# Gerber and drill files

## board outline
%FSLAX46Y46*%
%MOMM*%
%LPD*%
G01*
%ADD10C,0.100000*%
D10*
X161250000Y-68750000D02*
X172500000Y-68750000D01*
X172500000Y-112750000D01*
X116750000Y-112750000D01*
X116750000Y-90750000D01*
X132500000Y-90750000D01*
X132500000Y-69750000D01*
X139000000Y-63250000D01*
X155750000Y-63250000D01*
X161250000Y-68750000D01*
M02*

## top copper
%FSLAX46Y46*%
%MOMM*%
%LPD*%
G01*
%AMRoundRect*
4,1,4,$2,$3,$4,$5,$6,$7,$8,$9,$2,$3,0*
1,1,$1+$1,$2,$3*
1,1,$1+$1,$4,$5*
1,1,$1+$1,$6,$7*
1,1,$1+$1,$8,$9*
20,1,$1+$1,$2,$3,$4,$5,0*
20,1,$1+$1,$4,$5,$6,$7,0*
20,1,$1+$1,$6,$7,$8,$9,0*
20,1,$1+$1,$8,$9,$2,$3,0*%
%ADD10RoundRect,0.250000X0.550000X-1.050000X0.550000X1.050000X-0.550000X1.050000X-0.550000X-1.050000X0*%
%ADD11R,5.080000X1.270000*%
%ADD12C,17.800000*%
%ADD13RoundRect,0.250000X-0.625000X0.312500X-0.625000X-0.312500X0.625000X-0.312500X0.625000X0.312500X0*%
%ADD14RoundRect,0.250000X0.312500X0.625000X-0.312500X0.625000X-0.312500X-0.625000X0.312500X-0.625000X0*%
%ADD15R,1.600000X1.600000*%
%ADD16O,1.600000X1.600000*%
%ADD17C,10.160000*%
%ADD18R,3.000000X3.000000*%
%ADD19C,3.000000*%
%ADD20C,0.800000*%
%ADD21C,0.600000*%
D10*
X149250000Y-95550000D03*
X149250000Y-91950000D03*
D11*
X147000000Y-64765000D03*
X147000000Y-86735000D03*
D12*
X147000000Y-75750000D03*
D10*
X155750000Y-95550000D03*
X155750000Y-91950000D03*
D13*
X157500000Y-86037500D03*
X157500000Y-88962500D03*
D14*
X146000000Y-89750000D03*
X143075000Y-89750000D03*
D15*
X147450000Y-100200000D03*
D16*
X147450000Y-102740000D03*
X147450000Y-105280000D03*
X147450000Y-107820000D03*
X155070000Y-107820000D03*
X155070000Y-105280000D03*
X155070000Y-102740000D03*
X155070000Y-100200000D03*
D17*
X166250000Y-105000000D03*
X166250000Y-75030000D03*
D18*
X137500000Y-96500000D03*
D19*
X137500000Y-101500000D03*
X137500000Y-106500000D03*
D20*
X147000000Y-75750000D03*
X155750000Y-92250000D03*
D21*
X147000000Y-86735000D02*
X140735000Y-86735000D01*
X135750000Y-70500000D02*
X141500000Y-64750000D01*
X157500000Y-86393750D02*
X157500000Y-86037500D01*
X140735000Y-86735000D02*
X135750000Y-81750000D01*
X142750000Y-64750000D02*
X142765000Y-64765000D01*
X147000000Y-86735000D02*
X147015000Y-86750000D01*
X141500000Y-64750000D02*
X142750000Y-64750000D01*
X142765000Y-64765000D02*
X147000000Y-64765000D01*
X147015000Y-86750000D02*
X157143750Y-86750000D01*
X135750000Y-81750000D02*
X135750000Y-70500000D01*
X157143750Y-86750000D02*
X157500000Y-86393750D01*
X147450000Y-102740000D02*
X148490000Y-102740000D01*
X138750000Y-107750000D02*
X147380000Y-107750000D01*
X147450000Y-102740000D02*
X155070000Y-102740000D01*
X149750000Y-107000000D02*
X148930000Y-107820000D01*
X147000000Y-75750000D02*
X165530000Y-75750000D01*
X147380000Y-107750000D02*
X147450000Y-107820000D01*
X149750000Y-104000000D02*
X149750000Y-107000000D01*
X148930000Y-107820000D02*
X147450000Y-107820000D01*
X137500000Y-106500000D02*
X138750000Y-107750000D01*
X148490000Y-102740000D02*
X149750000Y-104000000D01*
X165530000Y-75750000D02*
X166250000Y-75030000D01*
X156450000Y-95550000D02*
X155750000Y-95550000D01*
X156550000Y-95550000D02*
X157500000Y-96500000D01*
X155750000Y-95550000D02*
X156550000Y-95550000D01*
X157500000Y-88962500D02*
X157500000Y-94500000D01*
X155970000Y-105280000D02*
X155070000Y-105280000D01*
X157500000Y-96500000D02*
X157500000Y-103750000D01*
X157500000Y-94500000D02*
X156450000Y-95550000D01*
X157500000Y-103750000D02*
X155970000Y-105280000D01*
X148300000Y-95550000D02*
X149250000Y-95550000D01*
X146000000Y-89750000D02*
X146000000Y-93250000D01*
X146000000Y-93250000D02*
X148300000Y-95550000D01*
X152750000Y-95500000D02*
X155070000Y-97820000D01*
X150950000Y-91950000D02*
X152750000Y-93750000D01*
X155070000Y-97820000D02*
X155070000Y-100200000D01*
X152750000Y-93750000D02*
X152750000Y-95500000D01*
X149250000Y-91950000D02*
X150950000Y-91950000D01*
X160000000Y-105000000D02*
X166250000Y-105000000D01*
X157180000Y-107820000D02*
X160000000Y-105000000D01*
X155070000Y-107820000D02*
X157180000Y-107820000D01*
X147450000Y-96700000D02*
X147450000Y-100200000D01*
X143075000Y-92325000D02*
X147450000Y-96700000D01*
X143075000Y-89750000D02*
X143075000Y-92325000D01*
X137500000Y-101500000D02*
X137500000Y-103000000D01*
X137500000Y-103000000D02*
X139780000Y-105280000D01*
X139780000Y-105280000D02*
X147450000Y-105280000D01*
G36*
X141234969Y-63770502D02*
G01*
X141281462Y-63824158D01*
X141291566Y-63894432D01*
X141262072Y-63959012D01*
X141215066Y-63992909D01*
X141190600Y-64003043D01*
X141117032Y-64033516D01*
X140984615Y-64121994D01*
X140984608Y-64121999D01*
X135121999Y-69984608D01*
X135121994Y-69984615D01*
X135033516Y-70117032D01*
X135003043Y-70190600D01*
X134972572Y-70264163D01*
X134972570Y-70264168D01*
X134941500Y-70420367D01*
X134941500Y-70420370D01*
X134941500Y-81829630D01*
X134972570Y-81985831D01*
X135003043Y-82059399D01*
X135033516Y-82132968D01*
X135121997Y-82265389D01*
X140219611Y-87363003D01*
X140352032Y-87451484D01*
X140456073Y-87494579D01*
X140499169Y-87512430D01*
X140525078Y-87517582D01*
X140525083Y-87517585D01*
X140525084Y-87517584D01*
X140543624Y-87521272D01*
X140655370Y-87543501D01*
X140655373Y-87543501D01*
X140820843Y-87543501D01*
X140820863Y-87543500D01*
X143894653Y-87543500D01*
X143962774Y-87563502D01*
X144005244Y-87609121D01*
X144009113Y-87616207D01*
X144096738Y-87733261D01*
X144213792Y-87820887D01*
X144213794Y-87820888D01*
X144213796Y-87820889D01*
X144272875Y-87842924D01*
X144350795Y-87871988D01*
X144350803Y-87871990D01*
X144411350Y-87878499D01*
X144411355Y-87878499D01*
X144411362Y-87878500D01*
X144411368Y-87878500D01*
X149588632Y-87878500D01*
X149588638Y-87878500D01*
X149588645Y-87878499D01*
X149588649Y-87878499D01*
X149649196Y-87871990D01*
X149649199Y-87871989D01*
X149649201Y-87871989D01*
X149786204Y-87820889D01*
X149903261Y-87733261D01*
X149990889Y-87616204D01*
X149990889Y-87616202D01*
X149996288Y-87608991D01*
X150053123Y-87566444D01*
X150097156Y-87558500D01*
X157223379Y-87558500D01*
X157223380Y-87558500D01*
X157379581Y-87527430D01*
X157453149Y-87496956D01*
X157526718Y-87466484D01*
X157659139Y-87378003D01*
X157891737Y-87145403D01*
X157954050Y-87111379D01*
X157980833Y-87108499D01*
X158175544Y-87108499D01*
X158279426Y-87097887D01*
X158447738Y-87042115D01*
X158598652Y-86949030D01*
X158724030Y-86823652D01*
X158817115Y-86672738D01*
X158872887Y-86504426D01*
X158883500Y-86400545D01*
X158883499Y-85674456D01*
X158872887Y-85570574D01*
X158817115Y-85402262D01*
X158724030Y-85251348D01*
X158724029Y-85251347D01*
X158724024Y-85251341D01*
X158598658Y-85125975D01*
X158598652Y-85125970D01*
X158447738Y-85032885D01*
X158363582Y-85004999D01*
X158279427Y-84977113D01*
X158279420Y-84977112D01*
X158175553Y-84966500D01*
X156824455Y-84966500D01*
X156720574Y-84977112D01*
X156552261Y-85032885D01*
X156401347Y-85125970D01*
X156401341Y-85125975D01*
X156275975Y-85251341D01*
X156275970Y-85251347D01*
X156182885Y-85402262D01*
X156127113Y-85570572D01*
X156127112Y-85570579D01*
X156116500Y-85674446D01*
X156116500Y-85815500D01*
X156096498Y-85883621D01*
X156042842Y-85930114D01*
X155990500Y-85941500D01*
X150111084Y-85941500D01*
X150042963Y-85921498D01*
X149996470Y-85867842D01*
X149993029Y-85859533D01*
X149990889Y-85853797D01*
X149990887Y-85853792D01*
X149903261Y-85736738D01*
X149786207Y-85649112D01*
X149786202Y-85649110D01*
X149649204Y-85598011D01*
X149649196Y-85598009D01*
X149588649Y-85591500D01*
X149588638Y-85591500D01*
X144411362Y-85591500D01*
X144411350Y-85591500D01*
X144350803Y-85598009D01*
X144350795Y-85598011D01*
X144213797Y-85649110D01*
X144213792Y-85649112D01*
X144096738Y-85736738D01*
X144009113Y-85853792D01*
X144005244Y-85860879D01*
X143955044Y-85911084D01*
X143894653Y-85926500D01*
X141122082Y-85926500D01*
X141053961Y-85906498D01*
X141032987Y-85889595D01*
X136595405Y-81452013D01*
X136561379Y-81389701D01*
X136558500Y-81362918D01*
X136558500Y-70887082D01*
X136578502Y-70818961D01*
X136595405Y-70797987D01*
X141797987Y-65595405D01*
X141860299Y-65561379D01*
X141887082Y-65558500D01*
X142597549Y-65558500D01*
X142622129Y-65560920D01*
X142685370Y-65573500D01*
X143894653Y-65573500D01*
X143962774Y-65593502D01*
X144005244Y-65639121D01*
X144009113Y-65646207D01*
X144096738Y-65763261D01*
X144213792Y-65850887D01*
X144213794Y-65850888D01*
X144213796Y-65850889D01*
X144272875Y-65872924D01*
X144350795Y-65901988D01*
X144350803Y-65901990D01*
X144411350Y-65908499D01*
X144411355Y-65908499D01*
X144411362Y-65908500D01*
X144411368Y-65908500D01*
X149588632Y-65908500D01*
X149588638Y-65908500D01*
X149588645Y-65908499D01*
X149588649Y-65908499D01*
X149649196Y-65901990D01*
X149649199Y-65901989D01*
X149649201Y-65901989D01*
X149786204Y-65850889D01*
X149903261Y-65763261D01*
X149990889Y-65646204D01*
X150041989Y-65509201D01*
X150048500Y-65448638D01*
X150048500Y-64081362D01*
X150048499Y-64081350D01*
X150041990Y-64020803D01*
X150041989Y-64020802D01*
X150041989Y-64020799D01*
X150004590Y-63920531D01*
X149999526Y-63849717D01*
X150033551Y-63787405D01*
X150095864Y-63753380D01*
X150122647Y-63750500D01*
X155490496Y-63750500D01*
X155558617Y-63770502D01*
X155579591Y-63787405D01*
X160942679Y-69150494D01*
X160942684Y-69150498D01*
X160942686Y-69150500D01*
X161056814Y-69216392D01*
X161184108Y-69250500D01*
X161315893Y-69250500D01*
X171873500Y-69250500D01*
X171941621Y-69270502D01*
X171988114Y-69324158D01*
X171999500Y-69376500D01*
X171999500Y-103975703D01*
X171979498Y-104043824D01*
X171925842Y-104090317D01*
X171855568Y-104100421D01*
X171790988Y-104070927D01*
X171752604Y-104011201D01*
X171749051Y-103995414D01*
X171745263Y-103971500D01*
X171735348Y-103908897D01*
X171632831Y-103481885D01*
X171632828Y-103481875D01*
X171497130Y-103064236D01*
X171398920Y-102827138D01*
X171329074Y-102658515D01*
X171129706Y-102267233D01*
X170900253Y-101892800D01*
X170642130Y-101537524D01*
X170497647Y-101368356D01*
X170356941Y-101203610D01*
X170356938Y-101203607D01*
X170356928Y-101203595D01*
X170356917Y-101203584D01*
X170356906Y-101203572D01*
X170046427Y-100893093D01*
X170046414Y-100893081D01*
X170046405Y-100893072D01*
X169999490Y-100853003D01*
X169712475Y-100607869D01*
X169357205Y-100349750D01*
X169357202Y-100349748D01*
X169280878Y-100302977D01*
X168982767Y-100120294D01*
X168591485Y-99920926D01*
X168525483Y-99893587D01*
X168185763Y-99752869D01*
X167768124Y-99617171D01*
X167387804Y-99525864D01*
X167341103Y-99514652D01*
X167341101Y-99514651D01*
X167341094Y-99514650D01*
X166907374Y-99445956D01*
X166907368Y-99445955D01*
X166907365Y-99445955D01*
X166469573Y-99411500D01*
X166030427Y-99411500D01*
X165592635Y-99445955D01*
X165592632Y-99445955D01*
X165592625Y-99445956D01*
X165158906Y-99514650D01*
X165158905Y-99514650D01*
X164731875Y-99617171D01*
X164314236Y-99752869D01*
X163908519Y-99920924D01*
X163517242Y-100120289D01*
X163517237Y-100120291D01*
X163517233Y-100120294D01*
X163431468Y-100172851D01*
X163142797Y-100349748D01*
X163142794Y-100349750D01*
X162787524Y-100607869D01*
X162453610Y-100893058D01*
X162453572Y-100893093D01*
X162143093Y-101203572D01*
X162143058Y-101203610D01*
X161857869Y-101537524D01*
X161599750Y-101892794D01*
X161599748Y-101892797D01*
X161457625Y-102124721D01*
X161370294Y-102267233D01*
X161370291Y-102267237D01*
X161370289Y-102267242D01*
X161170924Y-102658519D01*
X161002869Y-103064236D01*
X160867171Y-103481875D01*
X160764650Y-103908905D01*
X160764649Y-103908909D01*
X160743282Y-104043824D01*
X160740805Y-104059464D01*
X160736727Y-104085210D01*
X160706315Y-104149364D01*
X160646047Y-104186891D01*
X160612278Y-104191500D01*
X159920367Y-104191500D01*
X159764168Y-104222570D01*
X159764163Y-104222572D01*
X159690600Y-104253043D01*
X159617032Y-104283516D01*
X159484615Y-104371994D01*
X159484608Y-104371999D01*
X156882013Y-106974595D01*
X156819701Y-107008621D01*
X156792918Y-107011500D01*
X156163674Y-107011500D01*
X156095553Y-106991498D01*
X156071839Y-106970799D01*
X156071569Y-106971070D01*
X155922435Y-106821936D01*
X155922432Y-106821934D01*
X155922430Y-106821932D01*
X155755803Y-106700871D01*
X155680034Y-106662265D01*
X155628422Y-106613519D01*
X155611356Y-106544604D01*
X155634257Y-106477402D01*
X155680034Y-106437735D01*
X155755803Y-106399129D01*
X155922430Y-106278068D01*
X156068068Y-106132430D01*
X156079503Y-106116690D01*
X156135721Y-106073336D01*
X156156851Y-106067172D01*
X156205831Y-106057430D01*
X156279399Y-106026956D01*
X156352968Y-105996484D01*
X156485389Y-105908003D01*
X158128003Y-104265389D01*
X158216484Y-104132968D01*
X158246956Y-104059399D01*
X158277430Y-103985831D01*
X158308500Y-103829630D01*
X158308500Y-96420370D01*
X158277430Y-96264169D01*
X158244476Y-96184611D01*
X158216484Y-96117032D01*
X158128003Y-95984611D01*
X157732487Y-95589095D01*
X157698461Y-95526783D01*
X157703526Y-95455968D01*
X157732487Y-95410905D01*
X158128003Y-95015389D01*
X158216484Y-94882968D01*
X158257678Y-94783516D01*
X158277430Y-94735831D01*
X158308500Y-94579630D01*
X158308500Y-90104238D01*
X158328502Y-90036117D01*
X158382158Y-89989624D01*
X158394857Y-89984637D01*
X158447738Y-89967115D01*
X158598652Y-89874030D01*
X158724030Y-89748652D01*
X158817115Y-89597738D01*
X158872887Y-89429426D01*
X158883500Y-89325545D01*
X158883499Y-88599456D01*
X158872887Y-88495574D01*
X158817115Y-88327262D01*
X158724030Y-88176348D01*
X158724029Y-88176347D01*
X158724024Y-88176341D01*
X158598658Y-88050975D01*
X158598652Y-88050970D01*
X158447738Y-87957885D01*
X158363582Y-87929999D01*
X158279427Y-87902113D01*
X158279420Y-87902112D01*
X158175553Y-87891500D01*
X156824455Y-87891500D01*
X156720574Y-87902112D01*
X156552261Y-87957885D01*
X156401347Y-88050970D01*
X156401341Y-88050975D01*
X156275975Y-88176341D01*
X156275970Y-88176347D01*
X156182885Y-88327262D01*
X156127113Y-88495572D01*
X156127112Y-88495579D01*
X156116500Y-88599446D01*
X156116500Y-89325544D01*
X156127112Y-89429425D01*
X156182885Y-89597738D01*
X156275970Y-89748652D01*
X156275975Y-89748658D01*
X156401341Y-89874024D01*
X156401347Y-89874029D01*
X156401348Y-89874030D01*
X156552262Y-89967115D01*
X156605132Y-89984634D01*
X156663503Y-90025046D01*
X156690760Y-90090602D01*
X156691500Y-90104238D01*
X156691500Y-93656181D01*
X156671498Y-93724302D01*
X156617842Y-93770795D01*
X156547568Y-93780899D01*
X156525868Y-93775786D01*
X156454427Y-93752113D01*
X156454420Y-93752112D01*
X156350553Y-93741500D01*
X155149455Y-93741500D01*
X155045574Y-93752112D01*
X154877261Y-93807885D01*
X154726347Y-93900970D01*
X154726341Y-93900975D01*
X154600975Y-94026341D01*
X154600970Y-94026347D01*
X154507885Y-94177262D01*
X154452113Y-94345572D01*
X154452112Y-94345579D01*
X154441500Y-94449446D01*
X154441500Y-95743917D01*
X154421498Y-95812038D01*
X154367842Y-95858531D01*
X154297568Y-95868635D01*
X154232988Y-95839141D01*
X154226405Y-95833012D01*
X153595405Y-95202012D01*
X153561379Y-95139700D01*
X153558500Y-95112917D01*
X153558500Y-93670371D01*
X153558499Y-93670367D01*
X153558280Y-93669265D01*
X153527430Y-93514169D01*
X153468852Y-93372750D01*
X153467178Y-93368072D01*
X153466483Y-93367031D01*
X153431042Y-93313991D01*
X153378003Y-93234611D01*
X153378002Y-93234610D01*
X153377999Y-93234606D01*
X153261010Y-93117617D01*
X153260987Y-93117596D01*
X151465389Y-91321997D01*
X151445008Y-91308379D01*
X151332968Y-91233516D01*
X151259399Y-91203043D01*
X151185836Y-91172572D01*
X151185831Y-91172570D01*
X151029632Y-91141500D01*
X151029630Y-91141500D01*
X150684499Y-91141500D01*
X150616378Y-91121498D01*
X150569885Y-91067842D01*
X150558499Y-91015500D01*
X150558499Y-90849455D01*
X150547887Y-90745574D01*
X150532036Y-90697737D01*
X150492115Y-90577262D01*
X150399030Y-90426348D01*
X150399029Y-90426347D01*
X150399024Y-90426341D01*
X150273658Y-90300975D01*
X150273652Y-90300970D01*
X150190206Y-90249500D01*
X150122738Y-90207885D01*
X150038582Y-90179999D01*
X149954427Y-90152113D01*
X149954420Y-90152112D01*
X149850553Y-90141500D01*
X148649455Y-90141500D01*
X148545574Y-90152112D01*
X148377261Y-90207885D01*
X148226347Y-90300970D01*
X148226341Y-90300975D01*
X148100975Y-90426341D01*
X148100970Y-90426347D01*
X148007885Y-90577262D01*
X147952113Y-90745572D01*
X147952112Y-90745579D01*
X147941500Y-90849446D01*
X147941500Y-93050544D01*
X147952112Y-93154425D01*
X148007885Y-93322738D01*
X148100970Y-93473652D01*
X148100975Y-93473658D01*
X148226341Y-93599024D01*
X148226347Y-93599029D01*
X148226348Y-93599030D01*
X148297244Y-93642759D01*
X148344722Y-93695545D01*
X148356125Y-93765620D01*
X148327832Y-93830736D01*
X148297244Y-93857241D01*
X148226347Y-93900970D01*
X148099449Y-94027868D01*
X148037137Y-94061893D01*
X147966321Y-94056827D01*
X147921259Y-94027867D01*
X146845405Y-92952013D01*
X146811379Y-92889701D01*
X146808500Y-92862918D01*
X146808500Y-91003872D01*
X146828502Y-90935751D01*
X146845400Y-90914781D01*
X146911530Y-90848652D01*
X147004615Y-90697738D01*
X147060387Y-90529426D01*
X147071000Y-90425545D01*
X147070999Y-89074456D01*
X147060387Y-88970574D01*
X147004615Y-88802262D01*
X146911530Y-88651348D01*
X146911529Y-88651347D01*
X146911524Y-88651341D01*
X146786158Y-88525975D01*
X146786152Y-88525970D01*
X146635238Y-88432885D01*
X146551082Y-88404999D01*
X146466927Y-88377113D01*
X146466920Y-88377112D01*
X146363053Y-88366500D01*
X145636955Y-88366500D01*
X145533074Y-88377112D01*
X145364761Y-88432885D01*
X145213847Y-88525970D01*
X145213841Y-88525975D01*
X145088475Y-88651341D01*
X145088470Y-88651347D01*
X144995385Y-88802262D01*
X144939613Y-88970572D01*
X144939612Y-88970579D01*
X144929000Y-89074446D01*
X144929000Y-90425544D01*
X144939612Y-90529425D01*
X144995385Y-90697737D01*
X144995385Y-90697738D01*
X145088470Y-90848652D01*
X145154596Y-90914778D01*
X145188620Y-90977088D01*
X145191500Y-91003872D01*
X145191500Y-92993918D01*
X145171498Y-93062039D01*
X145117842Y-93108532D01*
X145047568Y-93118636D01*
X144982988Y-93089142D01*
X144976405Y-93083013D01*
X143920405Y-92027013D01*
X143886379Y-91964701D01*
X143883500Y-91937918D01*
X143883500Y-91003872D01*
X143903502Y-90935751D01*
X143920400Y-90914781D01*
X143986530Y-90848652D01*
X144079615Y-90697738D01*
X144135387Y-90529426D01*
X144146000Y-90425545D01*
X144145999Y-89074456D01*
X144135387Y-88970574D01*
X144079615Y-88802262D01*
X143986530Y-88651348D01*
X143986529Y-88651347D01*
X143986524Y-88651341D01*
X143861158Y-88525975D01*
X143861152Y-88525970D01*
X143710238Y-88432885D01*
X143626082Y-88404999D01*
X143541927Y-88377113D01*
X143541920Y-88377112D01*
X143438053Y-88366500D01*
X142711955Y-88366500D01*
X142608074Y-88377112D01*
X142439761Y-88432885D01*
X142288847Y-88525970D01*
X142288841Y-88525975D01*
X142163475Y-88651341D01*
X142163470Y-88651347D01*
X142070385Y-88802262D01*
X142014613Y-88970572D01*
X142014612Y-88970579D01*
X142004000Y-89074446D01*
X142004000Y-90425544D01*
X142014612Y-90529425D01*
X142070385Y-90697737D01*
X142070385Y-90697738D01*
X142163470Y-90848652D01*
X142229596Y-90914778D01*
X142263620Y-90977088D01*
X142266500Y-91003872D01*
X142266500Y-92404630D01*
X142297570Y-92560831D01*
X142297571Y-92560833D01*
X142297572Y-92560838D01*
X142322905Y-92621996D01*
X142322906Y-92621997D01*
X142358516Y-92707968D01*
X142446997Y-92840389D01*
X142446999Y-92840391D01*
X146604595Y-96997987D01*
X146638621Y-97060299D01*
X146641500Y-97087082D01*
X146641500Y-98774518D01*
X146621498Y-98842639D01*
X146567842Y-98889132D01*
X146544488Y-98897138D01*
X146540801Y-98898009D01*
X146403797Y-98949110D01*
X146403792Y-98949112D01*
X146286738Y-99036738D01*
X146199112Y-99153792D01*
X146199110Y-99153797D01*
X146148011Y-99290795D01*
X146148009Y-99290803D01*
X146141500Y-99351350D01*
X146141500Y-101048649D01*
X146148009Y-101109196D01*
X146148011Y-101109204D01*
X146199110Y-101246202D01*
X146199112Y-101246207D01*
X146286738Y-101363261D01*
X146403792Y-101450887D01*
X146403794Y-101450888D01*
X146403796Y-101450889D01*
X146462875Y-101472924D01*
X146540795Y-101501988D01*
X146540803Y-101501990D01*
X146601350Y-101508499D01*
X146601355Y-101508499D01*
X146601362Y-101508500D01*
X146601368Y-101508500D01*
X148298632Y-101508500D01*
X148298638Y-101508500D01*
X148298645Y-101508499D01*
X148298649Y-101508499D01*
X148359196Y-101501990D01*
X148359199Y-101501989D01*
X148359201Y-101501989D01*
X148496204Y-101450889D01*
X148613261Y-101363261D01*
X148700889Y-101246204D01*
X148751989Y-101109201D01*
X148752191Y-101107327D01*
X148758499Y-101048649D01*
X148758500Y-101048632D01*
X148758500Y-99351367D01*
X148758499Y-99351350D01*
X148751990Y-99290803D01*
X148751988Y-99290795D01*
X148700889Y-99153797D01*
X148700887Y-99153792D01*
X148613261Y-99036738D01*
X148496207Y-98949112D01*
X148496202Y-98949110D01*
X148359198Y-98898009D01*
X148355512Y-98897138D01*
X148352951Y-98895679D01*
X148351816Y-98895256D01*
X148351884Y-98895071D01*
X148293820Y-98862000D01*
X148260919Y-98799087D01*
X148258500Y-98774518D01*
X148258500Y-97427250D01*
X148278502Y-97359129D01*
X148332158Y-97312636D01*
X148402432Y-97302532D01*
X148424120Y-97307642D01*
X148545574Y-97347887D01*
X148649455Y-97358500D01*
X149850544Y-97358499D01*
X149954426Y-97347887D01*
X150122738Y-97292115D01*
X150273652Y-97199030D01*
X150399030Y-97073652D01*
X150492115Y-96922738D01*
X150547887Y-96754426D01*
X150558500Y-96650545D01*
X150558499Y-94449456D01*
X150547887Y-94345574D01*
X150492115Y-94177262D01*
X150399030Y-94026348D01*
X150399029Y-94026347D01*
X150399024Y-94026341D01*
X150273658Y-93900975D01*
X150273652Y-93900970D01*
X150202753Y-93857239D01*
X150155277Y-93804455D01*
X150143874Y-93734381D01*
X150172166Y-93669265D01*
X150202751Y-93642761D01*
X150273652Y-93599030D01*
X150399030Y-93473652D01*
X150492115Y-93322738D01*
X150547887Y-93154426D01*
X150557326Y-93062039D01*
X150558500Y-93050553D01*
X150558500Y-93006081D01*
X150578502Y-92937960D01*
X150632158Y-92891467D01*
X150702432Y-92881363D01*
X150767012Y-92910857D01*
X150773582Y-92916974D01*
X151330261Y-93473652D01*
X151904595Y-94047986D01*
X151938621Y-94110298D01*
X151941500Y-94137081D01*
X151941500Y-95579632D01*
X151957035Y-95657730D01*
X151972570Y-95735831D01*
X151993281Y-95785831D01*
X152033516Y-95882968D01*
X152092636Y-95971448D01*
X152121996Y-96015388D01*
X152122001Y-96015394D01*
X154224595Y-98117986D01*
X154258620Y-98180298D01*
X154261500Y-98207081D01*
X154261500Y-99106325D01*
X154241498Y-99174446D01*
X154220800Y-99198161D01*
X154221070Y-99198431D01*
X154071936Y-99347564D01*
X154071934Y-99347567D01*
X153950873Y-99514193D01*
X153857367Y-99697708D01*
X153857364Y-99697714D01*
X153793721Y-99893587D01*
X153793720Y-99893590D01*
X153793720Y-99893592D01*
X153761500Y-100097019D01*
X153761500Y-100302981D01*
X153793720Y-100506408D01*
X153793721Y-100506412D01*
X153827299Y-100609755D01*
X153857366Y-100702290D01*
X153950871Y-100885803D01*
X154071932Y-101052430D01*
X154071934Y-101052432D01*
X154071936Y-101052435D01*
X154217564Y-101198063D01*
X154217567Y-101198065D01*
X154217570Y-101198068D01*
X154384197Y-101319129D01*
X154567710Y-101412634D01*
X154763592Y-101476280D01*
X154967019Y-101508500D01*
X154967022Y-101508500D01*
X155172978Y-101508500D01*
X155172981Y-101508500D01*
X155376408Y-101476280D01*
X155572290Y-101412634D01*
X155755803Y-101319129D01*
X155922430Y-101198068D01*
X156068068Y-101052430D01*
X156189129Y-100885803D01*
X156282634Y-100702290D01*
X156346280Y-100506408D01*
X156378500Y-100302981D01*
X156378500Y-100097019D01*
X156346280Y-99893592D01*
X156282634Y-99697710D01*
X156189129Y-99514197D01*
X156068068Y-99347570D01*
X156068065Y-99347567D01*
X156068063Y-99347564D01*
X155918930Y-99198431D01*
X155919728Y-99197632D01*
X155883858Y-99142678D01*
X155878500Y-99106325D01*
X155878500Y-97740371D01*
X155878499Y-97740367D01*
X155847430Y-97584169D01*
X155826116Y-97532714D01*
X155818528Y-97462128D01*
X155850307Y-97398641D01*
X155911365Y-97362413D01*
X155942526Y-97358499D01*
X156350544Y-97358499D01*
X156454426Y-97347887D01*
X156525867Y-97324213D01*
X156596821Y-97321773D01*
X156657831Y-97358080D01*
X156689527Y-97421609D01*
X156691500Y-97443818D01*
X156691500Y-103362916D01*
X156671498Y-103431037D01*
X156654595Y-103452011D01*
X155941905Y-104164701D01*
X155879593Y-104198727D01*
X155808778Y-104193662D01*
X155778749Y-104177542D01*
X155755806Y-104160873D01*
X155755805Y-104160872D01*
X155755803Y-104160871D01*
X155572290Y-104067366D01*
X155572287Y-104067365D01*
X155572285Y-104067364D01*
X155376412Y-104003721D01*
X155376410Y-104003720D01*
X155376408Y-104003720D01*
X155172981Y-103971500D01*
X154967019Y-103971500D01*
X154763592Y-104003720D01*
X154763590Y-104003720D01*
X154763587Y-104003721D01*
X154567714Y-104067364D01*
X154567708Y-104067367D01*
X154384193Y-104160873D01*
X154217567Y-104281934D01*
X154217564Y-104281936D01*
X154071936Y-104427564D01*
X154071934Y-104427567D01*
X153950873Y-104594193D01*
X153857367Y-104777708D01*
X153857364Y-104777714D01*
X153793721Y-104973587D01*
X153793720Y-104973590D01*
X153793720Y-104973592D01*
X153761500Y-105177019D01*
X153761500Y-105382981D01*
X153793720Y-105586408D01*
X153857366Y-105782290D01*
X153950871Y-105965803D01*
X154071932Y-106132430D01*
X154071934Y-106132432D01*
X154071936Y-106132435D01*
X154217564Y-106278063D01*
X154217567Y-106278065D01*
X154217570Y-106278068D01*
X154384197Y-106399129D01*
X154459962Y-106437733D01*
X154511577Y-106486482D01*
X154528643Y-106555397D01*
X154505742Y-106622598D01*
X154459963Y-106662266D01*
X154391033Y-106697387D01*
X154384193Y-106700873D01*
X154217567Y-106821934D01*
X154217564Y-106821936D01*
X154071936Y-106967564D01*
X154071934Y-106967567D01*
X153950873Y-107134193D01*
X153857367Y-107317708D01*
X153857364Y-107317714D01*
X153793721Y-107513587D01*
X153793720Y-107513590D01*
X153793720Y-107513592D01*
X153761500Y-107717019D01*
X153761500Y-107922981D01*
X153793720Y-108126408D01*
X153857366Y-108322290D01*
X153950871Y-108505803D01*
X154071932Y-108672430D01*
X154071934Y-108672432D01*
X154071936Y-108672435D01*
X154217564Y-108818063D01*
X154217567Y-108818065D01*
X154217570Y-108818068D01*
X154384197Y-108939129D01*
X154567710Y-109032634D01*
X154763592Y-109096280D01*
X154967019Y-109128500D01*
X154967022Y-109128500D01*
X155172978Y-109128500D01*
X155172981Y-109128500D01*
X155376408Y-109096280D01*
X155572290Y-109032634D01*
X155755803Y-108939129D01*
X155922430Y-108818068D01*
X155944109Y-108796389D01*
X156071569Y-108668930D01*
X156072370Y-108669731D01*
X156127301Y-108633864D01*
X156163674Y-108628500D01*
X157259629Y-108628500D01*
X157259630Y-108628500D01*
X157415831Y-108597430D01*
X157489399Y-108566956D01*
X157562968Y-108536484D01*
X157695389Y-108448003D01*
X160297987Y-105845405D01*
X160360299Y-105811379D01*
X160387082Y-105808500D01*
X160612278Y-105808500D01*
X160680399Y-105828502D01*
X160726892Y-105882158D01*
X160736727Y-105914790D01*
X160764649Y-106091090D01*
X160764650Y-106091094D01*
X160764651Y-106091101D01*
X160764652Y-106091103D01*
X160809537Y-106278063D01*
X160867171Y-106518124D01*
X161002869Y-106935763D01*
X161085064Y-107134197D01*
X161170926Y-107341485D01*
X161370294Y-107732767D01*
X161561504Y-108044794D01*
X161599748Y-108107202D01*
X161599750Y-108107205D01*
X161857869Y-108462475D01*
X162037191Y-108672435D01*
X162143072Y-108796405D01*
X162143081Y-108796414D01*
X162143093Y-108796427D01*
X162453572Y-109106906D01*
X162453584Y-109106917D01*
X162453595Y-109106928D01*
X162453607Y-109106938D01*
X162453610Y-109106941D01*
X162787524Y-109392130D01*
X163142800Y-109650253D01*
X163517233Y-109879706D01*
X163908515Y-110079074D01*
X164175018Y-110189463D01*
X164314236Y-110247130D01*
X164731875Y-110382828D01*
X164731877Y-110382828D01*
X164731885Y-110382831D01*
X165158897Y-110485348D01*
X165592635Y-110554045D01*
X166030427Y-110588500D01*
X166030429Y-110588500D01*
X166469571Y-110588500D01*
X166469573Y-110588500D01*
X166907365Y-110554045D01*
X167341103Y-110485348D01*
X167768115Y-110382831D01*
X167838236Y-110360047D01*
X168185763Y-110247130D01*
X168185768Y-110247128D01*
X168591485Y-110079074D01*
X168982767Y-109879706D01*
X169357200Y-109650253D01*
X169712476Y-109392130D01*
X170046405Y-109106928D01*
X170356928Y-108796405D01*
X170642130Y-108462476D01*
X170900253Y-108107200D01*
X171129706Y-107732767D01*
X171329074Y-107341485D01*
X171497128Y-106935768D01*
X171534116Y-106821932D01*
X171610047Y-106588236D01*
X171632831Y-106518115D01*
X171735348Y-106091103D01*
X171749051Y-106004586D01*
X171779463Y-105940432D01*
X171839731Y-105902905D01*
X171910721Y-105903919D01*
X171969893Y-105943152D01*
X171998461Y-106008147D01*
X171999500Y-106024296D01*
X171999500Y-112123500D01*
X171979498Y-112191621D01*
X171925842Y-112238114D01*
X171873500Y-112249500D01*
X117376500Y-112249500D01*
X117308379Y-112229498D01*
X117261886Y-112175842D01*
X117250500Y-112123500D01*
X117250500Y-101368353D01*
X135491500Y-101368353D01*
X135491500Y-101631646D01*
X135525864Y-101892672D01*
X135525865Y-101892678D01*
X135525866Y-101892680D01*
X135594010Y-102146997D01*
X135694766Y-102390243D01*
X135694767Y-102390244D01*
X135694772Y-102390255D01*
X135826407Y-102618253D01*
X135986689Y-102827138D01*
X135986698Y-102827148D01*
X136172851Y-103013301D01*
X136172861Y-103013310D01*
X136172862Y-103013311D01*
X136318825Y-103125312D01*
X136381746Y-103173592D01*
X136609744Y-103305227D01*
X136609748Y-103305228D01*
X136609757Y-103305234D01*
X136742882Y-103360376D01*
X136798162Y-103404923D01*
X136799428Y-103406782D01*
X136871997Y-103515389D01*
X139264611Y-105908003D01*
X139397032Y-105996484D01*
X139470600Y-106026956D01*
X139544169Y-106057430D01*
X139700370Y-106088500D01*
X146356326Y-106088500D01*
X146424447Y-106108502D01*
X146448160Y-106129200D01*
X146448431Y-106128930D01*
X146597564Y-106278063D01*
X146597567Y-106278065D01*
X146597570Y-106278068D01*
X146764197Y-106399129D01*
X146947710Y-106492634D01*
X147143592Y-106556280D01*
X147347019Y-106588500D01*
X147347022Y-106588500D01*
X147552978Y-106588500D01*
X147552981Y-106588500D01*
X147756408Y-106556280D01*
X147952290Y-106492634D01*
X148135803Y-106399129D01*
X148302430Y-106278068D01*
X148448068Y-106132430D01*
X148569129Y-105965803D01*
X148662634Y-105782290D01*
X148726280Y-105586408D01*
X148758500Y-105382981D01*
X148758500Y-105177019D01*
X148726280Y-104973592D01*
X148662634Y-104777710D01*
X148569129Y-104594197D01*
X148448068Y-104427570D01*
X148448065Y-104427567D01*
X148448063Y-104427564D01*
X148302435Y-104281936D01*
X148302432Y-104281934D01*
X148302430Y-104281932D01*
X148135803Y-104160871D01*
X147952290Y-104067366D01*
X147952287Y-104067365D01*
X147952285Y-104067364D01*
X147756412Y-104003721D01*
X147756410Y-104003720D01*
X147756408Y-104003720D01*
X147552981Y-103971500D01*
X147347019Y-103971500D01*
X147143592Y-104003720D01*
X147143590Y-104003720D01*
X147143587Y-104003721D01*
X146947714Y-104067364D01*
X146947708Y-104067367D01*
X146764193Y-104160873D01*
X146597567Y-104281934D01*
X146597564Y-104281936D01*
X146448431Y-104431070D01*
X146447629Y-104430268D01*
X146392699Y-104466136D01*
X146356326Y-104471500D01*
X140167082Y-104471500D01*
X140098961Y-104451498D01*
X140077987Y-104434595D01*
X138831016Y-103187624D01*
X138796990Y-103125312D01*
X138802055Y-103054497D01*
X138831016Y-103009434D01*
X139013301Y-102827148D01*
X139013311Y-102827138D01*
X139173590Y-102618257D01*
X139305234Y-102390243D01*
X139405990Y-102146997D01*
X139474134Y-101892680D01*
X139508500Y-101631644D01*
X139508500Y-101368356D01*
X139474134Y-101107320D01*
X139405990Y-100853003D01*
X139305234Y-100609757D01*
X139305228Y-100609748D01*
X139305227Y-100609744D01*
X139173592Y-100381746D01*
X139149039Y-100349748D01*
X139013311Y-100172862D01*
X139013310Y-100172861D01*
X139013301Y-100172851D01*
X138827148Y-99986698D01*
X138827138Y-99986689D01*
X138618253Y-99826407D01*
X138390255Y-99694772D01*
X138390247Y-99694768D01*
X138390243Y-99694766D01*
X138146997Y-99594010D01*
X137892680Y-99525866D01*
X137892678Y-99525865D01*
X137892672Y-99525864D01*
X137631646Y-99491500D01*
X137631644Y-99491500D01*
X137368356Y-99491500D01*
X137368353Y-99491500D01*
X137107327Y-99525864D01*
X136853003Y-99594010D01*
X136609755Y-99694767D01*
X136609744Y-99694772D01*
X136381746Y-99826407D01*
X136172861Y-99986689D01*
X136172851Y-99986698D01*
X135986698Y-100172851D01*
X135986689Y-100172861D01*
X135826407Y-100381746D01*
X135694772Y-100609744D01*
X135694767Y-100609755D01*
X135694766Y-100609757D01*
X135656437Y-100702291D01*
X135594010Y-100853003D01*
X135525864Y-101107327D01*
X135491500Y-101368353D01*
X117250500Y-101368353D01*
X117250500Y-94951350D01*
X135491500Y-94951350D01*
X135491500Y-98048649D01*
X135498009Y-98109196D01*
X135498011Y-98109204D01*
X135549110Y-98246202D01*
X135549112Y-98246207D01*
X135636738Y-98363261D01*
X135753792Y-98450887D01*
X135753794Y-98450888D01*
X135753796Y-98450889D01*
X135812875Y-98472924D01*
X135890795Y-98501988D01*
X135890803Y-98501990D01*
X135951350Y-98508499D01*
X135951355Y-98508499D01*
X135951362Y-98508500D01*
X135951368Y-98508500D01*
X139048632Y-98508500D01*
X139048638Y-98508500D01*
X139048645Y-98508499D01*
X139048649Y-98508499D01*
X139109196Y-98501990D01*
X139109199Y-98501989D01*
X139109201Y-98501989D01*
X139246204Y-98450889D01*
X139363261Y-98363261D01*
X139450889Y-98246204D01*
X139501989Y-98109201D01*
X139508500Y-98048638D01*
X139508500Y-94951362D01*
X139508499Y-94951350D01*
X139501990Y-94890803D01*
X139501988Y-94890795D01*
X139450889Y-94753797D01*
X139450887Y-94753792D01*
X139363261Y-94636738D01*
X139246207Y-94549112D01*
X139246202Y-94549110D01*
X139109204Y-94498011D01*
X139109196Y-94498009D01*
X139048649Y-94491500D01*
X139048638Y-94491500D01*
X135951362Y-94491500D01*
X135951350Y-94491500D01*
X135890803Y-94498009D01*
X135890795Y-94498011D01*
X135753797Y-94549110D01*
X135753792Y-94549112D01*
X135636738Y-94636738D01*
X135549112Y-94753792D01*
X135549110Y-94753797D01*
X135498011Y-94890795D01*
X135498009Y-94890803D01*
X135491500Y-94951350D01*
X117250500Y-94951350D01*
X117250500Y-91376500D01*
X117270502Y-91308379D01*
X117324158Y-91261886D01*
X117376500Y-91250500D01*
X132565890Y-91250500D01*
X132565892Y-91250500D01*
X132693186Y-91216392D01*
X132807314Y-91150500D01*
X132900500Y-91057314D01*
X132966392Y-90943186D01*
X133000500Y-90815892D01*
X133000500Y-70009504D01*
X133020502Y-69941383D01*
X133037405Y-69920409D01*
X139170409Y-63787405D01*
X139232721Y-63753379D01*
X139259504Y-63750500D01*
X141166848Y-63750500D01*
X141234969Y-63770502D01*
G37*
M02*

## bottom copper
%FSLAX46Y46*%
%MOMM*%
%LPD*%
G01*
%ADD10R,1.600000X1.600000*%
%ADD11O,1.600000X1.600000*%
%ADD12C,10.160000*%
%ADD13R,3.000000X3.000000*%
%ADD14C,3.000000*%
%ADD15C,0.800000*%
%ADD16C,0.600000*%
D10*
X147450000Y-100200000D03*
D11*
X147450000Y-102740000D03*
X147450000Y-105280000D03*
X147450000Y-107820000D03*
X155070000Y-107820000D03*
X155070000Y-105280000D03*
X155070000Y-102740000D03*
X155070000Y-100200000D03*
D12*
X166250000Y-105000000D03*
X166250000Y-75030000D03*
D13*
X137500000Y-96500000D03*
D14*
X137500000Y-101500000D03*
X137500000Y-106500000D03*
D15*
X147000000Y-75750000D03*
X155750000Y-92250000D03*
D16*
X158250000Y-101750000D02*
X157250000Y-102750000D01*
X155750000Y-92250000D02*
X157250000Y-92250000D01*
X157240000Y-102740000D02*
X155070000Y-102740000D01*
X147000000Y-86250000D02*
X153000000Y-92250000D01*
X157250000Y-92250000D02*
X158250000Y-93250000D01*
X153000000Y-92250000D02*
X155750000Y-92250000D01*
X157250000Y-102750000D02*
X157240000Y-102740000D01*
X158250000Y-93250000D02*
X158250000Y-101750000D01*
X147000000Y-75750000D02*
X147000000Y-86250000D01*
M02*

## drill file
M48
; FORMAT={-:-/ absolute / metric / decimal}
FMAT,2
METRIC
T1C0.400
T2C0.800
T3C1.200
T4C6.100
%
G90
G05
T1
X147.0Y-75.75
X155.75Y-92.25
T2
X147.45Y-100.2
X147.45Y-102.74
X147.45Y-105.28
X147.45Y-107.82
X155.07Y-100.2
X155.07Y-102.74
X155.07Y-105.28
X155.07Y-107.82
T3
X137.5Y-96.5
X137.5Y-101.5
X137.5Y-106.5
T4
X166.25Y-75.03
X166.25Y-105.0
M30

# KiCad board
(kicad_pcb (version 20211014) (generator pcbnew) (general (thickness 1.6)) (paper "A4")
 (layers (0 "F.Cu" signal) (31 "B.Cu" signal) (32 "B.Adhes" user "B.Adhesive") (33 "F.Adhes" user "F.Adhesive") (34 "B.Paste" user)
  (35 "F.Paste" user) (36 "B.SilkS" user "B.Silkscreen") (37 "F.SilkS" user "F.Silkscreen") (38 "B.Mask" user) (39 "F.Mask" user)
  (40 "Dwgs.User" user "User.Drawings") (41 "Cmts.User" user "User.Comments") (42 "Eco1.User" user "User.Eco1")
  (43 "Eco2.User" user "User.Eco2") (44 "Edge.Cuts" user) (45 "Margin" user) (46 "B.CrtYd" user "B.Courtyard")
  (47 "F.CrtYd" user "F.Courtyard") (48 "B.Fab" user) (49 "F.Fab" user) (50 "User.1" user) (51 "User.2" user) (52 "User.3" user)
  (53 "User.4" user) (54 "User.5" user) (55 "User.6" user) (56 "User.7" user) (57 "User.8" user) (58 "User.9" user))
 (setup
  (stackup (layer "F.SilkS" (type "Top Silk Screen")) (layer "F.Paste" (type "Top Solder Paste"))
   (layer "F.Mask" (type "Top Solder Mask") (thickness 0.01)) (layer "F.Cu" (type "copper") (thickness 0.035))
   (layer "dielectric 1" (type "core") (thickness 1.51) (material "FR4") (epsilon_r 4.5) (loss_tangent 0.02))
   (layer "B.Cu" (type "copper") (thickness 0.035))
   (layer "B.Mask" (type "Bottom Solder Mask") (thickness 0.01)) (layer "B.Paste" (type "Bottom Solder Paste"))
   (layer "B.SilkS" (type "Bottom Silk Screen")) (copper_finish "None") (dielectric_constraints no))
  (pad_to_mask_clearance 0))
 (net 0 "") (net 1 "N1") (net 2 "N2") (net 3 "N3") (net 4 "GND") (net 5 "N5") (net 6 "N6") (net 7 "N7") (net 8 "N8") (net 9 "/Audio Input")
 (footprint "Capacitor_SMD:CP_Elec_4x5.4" (layer "F.Cu") (at 149.25 93.75 90)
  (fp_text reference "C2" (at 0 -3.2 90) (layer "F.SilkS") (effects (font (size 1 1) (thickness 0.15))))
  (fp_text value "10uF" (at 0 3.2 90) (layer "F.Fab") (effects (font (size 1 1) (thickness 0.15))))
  (pad "1" smd roundrect (at -1.8 0 90) (size 2.6 1.6) (layers "F.Cu" "F.Paste" "F.Mask") (roundrect_rratio 0.15625) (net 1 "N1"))
  (pad "2" smd roundrect (at 1.8 0 90) (size 2.6 1.6) (layers "F.Cu" "F.Paste" "F.Mask") (roundrect_rratio 0.15625) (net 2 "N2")))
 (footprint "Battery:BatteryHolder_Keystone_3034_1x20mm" (layer "F.Cu") (at 147 75.75 90)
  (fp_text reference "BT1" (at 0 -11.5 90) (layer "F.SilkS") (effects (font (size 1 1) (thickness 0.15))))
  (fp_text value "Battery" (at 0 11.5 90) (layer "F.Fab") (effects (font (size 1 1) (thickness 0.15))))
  (pad "1" smd rect (at 10.985 0 90) (size 1.27 5.08) (layers "F.Cu" "F.Paste" "F.Mask") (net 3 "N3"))
  (pad "1" smd rect (at -10.985 0 90) (size 1.27 5.08) (layers "F.Cu" "F.Paste" "F.Mask") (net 3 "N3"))
  (pad "2" smd circle (at 0 0 90) (size 17.8 17.8) (layers "F.Cu" "F.Mask") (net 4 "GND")))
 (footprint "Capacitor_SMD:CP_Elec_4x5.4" (layer "F.Cu") (at 155.75 93.75 90)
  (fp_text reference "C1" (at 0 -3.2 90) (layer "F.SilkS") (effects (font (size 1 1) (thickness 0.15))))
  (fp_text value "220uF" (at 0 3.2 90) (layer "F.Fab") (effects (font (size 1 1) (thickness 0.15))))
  (pad "1" smd roundrect (at -1.8 0 90) (size 2.6 1.6) (layers "F.Cu" "F.Paste" "F.Mask") (roundrect_rratio 0.15625) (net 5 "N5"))
  (pad "2" smd roundrect (at 1.8 0 90) (size 2.6 1.6) (layers "F.Cu" "F.Paste" "F.Mask") (roundrect_rratio 0.15625) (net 4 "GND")))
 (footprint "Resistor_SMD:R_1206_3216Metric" (layer "F.Cu") (at 157.5 87.5 -90)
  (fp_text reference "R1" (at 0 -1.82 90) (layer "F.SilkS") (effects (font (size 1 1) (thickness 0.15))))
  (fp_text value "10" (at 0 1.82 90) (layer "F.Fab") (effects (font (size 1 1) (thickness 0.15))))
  (pad "1" smd roundrect (at -1.4625 0 270) (size 1.125 1.75) (layers "F.Cu" "F.Paste" "F.Mask") (roundrect_rratio 0.2222222222)
   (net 3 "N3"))
  (pad "2" smd roundrect (at 1.4625 0 270) (size 1.125 1.75) (layers "F.Cu" "F.Paste" "F.Mask") (roundrect_rratio 0.2222222222) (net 5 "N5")))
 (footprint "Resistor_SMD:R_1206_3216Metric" (layer "F.Cu") (at 144.5375 89.75 180)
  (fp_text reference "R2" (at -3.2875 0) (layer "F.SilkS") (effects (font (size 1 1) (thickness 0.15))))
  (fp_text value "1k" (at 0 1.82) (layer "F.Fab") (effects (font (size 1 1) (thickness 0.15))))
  (pad "1" smd roundrect (at -1.4625 0 180) (size 1.125 1.75) (layers "F.Cu" "F.Paste" "F.Mask") (roundrect_rratio 0.2222222222)
   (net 1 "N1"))
  (pad "2" smd roundrect (at 1.4625 0 180) (size 1.125 1.75) (layers "F.Cu" "F.Paste" "F.Mask") (roundrect_rratio 0.2222222222) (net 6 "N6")))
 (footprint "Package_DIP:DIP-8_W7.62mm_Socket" (layer "F.Cu") (at 147.45 100.2)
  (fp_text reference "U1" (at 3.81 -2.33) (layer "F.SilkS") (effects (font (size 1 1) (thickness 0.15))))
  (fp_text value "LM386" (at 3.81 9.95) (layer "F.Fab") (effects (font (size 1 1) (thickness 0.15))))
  (pad "1" thru_hole rect (at 0 0) (size 1.6 1.6) (drill 0.8) (layers *.Cu *.Mask) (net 6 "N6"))
  (pad "2" thru_hole oval (at 0 2.54) (size 1.6 1.6) (drill 0.8) (layers *.Cu *.Mask) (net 4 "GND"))
  (pad "3" thru_hole oval (at 0 5.08) (size 1.6 1.6) (drill 0.8) (layers *.Cu *.Mask) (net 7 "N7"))
  (pad "4" thru_hole oval (at 0 7.62) (size 1.6 1.6) (drill 0.8) (layers *.Cu *.Mask) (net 4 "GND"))
  (pad "5" thru_hole oval (at 7.62 7.62) (size 1.6 1.6) (drill 0.8) (layers *.Cu *.Mask) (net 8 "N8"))
  (pad "6" thru_hole oval (at 7.62 5.08) (size 1.6 1.6) (drill 0.8) (layers *.Cu *.Mask) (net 5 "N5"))
  (pad "7" thru_hole oval (at 7.62 2.54) (size 1.6 1.6) (drill 0.8) (layers *.Cu *.Mask) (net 4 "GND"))
  (pad "8" thru_hole oval (at 7.62 0) (size 1.6 1.6) (drill 0.8) (layers *.Cu *.Mask) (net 2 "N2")))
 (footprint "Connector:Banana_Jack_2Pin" (layer "F.Cu") (at 166.25 105 90)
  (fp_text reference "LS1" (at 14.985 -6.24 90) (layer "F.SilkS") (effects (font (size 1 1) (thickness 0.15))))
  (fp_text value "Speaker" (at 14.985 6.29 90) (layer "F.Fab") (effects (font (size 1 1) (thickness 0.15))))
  (pad "1" thru_hole circle (at 0 0 90) (size 10.16 10.16) (drill 6.1) (layers *.Cu *.Mask) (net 8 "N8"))
  (pad "2" thru_hole circle (at 29.97 0 90) (size 10.16 10.16) (drill 6.1) (layers *.Cu *.Mask) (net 4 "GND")))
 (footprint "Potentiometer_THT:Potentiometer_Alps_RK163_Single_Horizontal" (layer "F.Cu") (at 137.5 96.5)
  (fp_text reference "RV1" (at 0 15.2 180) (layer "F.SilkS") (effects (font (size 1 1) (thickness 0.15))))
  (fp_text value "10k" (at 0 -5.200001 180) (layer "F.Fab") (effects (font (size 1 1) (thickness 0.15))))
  (pad "1" thru_hole rect (at 0 0 180) (size 3 3) (drill 1.2) (layers *.Cu *.Mask) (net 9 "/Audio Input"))
  (pad "2" thru_hole circle (at 0 5 180) (size 3 3) (drill 1.2) (layers *.Cu *.Mask) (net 7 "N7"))
  (pad "3" thru_hole circle (at 0 10 180) (size 3 3) (drill 1.2) (layers *.Cu *.Mask) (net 4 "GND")))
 (gr_poly
  (pts (xy 161.25 68.75) (xy 172.5 68.75) (xy 172.5 112.75) (xy 116.75 112.75) (xy 116.75 90.75) (xy 132.5 90.75) (xy 132.5 69.75)
   (xy 139 63.25) (xy 155.75 63.25))
  (layer "Edge.Cuts") (width 0.1) (fill none))
 (segment (start 147 86.735) (end 140.735 86.735) (width 0.6) (layer "F.Cu") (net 3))
 (segment (start 135.75 70.5) (end 141.5 64.75) (width 0.6) (layer "F.Cu") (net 3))
 (segment (start 157.5 86.39375) (end 157.5 86.0375) (width 0.6) (layer "F.Cu") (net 3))
 (segment (start 140.735 86.735) (end 135.75 81.75) (width 0.6) (layer "F.Cu") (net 3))
 (segment (start 142.75 64.75) (end 142.765 64.765) (width 0.6) (layer "F.Cu") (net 3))
 (segment (start 147 86.735) (end 147.015 86.75) (width 0.6) (layer "F.Cu") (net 3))
 (segment (start 141.5 64.75) (end 142.75 64.75) (width 0.6) (layer "F.Cu") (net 3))
 (segment (start 142.765 64.765) (end 147 64.765) (width 0.6) (layer "F.Cu") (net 3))
 (segment (start 147.015 86.75) (end 157.14375 86.75) (width 0.6) (layer "F.Cu") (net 3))
 (segment (start 135.75 81.75) (end 135.75 70.5) (width 0.6) (layer "F.Cu") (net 3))
 (segment (start 157.14375 86.75) (end 157.5 86.39375) (width 0.6) (layer "F.Cu") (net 3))
 (segment (start 147.45 102.74) (end 148.49 102.74) (width 0.6) (layer "F.Cu") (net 4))
 (segment (start 138.75 107.75) (end 147.38 107.75) (width 0.6) (layer "F.Cu") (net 4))
 (segment (start 147.45 102.74) (end 155.07 102.74) (width 0.6) (layer "F.Cu") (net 4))
 (segment (start 149.75 107) (end 148.93 107.82) (width 0.6) (layer "F.Cu") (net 4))
 (segment (start 147 75.75) (end 165.53 75.75) (width 0.6) (layer "F.Cu") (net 4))
 (segment (start 147.38 107.75) (end 147.45 107.82) (width 0.6) (layer "F.Cu") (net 4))
 (segment (start 149.75 104) (end 149.75 107) (width 0.6) (layer "F.Cu") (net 4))
 (segment (start 148.93 107.82) (end 147.45 107.82) (width 0.6) (layer "F.Cu") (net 4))
 (segment (start 137.5 106.5) (end 138.75 107.75) (width 0.6) (layer "F.Cu") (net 4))
 (segment (start 148.49 102.74) (end 149.75 104) (width 0.6) (layer "F.Cu") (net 4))
 (segment (start 165.53 75.75) (end 166.25 75.03) (width 0.6) (layer "F.Cu") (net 4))
 (via (at 147 75.75) (size 0.8) (drill 0.4) (layers "F.Cu" "B.Cu") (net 4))
 (via (at 155.75 92.25) (size 0.8) (drill 0.4) (layers "F.Cu" "B.Cu") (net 4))
 (segment (start 158.25 101.75) (end 157.25 102.75) (width 0.6) (layer "B.Cu") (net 4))
 (segment (start 155.75 92.25) (end 157.25 92.25) (width 0.6) (layer "B.Cu") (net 4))
 (segment (start 157.24 102.74) (end 155.07 102.74) (width 0.6) (layer "B.Cu") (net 4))
 (segment (start 147 86.25) (end 153 92.25) (width 0.6) (layer "B.Cu") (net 4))
 (segment (start 157.25 92.25) (end 158.25 93.25) (width 0.6) (layer "B.Cu") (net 4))
 (segment (start 153 92.25) (end 155.75 92.25) (width 0.6) (layer "B.Cu") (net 4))
 (segment (start 157.25 102.75) (end 157.24 102.74) (width 0.6) (layer "B.Cu") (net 4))
 (segment (start 158.25 93.25) (end 158.25 101.75) (width 0.6) (layer "B.Cu") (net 4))
 (segment (start 147 75.75) (end 147 86.25) (width 0.6) (layer "B.Cu") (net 4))
 (segment (start 156.45 95.55) (end 155.75 95.55) (width 0.6) (layer "F.Cu") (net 5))
 (segment (start 156.55 95.55) (end 157.5 96.5) (width 0.6) (layer "F.Cu") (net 5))
 (segment (start 155.75 95.55) (end 156.55 95.55) (width 0.6) (layer "F.Cu") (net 5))
 (segment (start 157.5 88.9625) (end 157.5 94.5) (width 0.6) (layer "F.Cu") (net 5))
 (segment (start 155.97 105.28) (end 155.07 105.28) (width 0.6) (layer "F.Cu") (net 5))
 (segment (start 157.5 96.5) (end 157.5 103.75) (width 0.6) (layer "F.Cu") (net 5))
 (segment (start 157.5 94.5) (end 156.45 95.55) (width 0.6) (layer "F.Cu") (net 5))
 (segment (start 157.5 103.75) (end 155.97 105.28) (width 0.6) (layer "F.Cu") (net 5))
 (segment (start 148.3 95.55) (end 149.25 95.55) (width 0.6) (layer "F.Cu") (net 1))
 (segment (start 146 89.75) (end 146 93.25) (width 0.6) (layer "F.Cu") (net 1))
 (segment (start 146 93.25) (end 148.3 95.55) (width 0.6) (layer "F.Cu") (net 1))
 (segment (start 152.75 95.5) (end 155.07 97.82) (width 0.6) (layer "F.Cu") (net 2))
 (segment (start 150.95 91.95) (end 152.75 93.75) (width 0.6) (layer "F.Cu") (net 2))
 (segment (start 155.07 97.82) (end 155.07 100.2) (width 0.6) (layer "F.Cu") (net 2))
 (segment (start 152.75 93.75) (end 152.75 95.5) (width 0.6) (layer "F.Cu") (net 2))
 (segment (start 149.25 91.95) (end 150.95 91.95) (width 0.6) (layer "F.Cu") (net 2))
 (segment (start 160 105) (end 166.25 105) (width 0.6) (layer "F.Cu") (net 8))
 (segment (start 157.18 107.82) (end 160 105) (width 0.6) (layer "F.Cu") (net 8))
 (segment (start 155.07 107.82) (end 157.18 107.82) (width 0.6) (layer "F.Cu") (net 8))
 (segment (start 147.45 96.7) (end 147.45 100.2) (width 0.6) (layer "F.Cu") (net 6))
 (segment (start 143.075 92.325) (end 147.45 96.7) (width 0.6) (layer "F.Cu") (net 6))
 (segment (start 143.075 89.75) (end 143.075 92.325) (width 0.6) (layer "F.Cu") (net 6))
 (segment (start 137.5 101.5) (end 137.5 103) (width 0.6) (layer "F.Cu") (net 7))
 (segment (start 137.5 103) (end 139.78 105.28) (width 0.6) (layer "F.Cu") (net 7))
 (segment (start 139.78 105.28) (end 147.45 105.28) (width 0.6) (layer "F.Cu") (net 7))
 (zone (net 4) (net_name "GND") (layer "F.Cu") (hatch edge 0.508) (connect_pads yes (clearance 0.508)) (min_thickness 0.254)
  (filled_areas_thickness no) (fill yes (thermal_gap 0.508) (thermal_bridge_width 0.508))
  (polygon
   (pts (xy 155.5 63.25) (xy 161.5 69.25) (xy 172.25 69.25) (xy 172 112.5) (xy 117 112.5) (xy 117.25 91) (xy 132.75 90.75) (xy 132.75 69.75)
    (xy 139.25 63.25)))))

